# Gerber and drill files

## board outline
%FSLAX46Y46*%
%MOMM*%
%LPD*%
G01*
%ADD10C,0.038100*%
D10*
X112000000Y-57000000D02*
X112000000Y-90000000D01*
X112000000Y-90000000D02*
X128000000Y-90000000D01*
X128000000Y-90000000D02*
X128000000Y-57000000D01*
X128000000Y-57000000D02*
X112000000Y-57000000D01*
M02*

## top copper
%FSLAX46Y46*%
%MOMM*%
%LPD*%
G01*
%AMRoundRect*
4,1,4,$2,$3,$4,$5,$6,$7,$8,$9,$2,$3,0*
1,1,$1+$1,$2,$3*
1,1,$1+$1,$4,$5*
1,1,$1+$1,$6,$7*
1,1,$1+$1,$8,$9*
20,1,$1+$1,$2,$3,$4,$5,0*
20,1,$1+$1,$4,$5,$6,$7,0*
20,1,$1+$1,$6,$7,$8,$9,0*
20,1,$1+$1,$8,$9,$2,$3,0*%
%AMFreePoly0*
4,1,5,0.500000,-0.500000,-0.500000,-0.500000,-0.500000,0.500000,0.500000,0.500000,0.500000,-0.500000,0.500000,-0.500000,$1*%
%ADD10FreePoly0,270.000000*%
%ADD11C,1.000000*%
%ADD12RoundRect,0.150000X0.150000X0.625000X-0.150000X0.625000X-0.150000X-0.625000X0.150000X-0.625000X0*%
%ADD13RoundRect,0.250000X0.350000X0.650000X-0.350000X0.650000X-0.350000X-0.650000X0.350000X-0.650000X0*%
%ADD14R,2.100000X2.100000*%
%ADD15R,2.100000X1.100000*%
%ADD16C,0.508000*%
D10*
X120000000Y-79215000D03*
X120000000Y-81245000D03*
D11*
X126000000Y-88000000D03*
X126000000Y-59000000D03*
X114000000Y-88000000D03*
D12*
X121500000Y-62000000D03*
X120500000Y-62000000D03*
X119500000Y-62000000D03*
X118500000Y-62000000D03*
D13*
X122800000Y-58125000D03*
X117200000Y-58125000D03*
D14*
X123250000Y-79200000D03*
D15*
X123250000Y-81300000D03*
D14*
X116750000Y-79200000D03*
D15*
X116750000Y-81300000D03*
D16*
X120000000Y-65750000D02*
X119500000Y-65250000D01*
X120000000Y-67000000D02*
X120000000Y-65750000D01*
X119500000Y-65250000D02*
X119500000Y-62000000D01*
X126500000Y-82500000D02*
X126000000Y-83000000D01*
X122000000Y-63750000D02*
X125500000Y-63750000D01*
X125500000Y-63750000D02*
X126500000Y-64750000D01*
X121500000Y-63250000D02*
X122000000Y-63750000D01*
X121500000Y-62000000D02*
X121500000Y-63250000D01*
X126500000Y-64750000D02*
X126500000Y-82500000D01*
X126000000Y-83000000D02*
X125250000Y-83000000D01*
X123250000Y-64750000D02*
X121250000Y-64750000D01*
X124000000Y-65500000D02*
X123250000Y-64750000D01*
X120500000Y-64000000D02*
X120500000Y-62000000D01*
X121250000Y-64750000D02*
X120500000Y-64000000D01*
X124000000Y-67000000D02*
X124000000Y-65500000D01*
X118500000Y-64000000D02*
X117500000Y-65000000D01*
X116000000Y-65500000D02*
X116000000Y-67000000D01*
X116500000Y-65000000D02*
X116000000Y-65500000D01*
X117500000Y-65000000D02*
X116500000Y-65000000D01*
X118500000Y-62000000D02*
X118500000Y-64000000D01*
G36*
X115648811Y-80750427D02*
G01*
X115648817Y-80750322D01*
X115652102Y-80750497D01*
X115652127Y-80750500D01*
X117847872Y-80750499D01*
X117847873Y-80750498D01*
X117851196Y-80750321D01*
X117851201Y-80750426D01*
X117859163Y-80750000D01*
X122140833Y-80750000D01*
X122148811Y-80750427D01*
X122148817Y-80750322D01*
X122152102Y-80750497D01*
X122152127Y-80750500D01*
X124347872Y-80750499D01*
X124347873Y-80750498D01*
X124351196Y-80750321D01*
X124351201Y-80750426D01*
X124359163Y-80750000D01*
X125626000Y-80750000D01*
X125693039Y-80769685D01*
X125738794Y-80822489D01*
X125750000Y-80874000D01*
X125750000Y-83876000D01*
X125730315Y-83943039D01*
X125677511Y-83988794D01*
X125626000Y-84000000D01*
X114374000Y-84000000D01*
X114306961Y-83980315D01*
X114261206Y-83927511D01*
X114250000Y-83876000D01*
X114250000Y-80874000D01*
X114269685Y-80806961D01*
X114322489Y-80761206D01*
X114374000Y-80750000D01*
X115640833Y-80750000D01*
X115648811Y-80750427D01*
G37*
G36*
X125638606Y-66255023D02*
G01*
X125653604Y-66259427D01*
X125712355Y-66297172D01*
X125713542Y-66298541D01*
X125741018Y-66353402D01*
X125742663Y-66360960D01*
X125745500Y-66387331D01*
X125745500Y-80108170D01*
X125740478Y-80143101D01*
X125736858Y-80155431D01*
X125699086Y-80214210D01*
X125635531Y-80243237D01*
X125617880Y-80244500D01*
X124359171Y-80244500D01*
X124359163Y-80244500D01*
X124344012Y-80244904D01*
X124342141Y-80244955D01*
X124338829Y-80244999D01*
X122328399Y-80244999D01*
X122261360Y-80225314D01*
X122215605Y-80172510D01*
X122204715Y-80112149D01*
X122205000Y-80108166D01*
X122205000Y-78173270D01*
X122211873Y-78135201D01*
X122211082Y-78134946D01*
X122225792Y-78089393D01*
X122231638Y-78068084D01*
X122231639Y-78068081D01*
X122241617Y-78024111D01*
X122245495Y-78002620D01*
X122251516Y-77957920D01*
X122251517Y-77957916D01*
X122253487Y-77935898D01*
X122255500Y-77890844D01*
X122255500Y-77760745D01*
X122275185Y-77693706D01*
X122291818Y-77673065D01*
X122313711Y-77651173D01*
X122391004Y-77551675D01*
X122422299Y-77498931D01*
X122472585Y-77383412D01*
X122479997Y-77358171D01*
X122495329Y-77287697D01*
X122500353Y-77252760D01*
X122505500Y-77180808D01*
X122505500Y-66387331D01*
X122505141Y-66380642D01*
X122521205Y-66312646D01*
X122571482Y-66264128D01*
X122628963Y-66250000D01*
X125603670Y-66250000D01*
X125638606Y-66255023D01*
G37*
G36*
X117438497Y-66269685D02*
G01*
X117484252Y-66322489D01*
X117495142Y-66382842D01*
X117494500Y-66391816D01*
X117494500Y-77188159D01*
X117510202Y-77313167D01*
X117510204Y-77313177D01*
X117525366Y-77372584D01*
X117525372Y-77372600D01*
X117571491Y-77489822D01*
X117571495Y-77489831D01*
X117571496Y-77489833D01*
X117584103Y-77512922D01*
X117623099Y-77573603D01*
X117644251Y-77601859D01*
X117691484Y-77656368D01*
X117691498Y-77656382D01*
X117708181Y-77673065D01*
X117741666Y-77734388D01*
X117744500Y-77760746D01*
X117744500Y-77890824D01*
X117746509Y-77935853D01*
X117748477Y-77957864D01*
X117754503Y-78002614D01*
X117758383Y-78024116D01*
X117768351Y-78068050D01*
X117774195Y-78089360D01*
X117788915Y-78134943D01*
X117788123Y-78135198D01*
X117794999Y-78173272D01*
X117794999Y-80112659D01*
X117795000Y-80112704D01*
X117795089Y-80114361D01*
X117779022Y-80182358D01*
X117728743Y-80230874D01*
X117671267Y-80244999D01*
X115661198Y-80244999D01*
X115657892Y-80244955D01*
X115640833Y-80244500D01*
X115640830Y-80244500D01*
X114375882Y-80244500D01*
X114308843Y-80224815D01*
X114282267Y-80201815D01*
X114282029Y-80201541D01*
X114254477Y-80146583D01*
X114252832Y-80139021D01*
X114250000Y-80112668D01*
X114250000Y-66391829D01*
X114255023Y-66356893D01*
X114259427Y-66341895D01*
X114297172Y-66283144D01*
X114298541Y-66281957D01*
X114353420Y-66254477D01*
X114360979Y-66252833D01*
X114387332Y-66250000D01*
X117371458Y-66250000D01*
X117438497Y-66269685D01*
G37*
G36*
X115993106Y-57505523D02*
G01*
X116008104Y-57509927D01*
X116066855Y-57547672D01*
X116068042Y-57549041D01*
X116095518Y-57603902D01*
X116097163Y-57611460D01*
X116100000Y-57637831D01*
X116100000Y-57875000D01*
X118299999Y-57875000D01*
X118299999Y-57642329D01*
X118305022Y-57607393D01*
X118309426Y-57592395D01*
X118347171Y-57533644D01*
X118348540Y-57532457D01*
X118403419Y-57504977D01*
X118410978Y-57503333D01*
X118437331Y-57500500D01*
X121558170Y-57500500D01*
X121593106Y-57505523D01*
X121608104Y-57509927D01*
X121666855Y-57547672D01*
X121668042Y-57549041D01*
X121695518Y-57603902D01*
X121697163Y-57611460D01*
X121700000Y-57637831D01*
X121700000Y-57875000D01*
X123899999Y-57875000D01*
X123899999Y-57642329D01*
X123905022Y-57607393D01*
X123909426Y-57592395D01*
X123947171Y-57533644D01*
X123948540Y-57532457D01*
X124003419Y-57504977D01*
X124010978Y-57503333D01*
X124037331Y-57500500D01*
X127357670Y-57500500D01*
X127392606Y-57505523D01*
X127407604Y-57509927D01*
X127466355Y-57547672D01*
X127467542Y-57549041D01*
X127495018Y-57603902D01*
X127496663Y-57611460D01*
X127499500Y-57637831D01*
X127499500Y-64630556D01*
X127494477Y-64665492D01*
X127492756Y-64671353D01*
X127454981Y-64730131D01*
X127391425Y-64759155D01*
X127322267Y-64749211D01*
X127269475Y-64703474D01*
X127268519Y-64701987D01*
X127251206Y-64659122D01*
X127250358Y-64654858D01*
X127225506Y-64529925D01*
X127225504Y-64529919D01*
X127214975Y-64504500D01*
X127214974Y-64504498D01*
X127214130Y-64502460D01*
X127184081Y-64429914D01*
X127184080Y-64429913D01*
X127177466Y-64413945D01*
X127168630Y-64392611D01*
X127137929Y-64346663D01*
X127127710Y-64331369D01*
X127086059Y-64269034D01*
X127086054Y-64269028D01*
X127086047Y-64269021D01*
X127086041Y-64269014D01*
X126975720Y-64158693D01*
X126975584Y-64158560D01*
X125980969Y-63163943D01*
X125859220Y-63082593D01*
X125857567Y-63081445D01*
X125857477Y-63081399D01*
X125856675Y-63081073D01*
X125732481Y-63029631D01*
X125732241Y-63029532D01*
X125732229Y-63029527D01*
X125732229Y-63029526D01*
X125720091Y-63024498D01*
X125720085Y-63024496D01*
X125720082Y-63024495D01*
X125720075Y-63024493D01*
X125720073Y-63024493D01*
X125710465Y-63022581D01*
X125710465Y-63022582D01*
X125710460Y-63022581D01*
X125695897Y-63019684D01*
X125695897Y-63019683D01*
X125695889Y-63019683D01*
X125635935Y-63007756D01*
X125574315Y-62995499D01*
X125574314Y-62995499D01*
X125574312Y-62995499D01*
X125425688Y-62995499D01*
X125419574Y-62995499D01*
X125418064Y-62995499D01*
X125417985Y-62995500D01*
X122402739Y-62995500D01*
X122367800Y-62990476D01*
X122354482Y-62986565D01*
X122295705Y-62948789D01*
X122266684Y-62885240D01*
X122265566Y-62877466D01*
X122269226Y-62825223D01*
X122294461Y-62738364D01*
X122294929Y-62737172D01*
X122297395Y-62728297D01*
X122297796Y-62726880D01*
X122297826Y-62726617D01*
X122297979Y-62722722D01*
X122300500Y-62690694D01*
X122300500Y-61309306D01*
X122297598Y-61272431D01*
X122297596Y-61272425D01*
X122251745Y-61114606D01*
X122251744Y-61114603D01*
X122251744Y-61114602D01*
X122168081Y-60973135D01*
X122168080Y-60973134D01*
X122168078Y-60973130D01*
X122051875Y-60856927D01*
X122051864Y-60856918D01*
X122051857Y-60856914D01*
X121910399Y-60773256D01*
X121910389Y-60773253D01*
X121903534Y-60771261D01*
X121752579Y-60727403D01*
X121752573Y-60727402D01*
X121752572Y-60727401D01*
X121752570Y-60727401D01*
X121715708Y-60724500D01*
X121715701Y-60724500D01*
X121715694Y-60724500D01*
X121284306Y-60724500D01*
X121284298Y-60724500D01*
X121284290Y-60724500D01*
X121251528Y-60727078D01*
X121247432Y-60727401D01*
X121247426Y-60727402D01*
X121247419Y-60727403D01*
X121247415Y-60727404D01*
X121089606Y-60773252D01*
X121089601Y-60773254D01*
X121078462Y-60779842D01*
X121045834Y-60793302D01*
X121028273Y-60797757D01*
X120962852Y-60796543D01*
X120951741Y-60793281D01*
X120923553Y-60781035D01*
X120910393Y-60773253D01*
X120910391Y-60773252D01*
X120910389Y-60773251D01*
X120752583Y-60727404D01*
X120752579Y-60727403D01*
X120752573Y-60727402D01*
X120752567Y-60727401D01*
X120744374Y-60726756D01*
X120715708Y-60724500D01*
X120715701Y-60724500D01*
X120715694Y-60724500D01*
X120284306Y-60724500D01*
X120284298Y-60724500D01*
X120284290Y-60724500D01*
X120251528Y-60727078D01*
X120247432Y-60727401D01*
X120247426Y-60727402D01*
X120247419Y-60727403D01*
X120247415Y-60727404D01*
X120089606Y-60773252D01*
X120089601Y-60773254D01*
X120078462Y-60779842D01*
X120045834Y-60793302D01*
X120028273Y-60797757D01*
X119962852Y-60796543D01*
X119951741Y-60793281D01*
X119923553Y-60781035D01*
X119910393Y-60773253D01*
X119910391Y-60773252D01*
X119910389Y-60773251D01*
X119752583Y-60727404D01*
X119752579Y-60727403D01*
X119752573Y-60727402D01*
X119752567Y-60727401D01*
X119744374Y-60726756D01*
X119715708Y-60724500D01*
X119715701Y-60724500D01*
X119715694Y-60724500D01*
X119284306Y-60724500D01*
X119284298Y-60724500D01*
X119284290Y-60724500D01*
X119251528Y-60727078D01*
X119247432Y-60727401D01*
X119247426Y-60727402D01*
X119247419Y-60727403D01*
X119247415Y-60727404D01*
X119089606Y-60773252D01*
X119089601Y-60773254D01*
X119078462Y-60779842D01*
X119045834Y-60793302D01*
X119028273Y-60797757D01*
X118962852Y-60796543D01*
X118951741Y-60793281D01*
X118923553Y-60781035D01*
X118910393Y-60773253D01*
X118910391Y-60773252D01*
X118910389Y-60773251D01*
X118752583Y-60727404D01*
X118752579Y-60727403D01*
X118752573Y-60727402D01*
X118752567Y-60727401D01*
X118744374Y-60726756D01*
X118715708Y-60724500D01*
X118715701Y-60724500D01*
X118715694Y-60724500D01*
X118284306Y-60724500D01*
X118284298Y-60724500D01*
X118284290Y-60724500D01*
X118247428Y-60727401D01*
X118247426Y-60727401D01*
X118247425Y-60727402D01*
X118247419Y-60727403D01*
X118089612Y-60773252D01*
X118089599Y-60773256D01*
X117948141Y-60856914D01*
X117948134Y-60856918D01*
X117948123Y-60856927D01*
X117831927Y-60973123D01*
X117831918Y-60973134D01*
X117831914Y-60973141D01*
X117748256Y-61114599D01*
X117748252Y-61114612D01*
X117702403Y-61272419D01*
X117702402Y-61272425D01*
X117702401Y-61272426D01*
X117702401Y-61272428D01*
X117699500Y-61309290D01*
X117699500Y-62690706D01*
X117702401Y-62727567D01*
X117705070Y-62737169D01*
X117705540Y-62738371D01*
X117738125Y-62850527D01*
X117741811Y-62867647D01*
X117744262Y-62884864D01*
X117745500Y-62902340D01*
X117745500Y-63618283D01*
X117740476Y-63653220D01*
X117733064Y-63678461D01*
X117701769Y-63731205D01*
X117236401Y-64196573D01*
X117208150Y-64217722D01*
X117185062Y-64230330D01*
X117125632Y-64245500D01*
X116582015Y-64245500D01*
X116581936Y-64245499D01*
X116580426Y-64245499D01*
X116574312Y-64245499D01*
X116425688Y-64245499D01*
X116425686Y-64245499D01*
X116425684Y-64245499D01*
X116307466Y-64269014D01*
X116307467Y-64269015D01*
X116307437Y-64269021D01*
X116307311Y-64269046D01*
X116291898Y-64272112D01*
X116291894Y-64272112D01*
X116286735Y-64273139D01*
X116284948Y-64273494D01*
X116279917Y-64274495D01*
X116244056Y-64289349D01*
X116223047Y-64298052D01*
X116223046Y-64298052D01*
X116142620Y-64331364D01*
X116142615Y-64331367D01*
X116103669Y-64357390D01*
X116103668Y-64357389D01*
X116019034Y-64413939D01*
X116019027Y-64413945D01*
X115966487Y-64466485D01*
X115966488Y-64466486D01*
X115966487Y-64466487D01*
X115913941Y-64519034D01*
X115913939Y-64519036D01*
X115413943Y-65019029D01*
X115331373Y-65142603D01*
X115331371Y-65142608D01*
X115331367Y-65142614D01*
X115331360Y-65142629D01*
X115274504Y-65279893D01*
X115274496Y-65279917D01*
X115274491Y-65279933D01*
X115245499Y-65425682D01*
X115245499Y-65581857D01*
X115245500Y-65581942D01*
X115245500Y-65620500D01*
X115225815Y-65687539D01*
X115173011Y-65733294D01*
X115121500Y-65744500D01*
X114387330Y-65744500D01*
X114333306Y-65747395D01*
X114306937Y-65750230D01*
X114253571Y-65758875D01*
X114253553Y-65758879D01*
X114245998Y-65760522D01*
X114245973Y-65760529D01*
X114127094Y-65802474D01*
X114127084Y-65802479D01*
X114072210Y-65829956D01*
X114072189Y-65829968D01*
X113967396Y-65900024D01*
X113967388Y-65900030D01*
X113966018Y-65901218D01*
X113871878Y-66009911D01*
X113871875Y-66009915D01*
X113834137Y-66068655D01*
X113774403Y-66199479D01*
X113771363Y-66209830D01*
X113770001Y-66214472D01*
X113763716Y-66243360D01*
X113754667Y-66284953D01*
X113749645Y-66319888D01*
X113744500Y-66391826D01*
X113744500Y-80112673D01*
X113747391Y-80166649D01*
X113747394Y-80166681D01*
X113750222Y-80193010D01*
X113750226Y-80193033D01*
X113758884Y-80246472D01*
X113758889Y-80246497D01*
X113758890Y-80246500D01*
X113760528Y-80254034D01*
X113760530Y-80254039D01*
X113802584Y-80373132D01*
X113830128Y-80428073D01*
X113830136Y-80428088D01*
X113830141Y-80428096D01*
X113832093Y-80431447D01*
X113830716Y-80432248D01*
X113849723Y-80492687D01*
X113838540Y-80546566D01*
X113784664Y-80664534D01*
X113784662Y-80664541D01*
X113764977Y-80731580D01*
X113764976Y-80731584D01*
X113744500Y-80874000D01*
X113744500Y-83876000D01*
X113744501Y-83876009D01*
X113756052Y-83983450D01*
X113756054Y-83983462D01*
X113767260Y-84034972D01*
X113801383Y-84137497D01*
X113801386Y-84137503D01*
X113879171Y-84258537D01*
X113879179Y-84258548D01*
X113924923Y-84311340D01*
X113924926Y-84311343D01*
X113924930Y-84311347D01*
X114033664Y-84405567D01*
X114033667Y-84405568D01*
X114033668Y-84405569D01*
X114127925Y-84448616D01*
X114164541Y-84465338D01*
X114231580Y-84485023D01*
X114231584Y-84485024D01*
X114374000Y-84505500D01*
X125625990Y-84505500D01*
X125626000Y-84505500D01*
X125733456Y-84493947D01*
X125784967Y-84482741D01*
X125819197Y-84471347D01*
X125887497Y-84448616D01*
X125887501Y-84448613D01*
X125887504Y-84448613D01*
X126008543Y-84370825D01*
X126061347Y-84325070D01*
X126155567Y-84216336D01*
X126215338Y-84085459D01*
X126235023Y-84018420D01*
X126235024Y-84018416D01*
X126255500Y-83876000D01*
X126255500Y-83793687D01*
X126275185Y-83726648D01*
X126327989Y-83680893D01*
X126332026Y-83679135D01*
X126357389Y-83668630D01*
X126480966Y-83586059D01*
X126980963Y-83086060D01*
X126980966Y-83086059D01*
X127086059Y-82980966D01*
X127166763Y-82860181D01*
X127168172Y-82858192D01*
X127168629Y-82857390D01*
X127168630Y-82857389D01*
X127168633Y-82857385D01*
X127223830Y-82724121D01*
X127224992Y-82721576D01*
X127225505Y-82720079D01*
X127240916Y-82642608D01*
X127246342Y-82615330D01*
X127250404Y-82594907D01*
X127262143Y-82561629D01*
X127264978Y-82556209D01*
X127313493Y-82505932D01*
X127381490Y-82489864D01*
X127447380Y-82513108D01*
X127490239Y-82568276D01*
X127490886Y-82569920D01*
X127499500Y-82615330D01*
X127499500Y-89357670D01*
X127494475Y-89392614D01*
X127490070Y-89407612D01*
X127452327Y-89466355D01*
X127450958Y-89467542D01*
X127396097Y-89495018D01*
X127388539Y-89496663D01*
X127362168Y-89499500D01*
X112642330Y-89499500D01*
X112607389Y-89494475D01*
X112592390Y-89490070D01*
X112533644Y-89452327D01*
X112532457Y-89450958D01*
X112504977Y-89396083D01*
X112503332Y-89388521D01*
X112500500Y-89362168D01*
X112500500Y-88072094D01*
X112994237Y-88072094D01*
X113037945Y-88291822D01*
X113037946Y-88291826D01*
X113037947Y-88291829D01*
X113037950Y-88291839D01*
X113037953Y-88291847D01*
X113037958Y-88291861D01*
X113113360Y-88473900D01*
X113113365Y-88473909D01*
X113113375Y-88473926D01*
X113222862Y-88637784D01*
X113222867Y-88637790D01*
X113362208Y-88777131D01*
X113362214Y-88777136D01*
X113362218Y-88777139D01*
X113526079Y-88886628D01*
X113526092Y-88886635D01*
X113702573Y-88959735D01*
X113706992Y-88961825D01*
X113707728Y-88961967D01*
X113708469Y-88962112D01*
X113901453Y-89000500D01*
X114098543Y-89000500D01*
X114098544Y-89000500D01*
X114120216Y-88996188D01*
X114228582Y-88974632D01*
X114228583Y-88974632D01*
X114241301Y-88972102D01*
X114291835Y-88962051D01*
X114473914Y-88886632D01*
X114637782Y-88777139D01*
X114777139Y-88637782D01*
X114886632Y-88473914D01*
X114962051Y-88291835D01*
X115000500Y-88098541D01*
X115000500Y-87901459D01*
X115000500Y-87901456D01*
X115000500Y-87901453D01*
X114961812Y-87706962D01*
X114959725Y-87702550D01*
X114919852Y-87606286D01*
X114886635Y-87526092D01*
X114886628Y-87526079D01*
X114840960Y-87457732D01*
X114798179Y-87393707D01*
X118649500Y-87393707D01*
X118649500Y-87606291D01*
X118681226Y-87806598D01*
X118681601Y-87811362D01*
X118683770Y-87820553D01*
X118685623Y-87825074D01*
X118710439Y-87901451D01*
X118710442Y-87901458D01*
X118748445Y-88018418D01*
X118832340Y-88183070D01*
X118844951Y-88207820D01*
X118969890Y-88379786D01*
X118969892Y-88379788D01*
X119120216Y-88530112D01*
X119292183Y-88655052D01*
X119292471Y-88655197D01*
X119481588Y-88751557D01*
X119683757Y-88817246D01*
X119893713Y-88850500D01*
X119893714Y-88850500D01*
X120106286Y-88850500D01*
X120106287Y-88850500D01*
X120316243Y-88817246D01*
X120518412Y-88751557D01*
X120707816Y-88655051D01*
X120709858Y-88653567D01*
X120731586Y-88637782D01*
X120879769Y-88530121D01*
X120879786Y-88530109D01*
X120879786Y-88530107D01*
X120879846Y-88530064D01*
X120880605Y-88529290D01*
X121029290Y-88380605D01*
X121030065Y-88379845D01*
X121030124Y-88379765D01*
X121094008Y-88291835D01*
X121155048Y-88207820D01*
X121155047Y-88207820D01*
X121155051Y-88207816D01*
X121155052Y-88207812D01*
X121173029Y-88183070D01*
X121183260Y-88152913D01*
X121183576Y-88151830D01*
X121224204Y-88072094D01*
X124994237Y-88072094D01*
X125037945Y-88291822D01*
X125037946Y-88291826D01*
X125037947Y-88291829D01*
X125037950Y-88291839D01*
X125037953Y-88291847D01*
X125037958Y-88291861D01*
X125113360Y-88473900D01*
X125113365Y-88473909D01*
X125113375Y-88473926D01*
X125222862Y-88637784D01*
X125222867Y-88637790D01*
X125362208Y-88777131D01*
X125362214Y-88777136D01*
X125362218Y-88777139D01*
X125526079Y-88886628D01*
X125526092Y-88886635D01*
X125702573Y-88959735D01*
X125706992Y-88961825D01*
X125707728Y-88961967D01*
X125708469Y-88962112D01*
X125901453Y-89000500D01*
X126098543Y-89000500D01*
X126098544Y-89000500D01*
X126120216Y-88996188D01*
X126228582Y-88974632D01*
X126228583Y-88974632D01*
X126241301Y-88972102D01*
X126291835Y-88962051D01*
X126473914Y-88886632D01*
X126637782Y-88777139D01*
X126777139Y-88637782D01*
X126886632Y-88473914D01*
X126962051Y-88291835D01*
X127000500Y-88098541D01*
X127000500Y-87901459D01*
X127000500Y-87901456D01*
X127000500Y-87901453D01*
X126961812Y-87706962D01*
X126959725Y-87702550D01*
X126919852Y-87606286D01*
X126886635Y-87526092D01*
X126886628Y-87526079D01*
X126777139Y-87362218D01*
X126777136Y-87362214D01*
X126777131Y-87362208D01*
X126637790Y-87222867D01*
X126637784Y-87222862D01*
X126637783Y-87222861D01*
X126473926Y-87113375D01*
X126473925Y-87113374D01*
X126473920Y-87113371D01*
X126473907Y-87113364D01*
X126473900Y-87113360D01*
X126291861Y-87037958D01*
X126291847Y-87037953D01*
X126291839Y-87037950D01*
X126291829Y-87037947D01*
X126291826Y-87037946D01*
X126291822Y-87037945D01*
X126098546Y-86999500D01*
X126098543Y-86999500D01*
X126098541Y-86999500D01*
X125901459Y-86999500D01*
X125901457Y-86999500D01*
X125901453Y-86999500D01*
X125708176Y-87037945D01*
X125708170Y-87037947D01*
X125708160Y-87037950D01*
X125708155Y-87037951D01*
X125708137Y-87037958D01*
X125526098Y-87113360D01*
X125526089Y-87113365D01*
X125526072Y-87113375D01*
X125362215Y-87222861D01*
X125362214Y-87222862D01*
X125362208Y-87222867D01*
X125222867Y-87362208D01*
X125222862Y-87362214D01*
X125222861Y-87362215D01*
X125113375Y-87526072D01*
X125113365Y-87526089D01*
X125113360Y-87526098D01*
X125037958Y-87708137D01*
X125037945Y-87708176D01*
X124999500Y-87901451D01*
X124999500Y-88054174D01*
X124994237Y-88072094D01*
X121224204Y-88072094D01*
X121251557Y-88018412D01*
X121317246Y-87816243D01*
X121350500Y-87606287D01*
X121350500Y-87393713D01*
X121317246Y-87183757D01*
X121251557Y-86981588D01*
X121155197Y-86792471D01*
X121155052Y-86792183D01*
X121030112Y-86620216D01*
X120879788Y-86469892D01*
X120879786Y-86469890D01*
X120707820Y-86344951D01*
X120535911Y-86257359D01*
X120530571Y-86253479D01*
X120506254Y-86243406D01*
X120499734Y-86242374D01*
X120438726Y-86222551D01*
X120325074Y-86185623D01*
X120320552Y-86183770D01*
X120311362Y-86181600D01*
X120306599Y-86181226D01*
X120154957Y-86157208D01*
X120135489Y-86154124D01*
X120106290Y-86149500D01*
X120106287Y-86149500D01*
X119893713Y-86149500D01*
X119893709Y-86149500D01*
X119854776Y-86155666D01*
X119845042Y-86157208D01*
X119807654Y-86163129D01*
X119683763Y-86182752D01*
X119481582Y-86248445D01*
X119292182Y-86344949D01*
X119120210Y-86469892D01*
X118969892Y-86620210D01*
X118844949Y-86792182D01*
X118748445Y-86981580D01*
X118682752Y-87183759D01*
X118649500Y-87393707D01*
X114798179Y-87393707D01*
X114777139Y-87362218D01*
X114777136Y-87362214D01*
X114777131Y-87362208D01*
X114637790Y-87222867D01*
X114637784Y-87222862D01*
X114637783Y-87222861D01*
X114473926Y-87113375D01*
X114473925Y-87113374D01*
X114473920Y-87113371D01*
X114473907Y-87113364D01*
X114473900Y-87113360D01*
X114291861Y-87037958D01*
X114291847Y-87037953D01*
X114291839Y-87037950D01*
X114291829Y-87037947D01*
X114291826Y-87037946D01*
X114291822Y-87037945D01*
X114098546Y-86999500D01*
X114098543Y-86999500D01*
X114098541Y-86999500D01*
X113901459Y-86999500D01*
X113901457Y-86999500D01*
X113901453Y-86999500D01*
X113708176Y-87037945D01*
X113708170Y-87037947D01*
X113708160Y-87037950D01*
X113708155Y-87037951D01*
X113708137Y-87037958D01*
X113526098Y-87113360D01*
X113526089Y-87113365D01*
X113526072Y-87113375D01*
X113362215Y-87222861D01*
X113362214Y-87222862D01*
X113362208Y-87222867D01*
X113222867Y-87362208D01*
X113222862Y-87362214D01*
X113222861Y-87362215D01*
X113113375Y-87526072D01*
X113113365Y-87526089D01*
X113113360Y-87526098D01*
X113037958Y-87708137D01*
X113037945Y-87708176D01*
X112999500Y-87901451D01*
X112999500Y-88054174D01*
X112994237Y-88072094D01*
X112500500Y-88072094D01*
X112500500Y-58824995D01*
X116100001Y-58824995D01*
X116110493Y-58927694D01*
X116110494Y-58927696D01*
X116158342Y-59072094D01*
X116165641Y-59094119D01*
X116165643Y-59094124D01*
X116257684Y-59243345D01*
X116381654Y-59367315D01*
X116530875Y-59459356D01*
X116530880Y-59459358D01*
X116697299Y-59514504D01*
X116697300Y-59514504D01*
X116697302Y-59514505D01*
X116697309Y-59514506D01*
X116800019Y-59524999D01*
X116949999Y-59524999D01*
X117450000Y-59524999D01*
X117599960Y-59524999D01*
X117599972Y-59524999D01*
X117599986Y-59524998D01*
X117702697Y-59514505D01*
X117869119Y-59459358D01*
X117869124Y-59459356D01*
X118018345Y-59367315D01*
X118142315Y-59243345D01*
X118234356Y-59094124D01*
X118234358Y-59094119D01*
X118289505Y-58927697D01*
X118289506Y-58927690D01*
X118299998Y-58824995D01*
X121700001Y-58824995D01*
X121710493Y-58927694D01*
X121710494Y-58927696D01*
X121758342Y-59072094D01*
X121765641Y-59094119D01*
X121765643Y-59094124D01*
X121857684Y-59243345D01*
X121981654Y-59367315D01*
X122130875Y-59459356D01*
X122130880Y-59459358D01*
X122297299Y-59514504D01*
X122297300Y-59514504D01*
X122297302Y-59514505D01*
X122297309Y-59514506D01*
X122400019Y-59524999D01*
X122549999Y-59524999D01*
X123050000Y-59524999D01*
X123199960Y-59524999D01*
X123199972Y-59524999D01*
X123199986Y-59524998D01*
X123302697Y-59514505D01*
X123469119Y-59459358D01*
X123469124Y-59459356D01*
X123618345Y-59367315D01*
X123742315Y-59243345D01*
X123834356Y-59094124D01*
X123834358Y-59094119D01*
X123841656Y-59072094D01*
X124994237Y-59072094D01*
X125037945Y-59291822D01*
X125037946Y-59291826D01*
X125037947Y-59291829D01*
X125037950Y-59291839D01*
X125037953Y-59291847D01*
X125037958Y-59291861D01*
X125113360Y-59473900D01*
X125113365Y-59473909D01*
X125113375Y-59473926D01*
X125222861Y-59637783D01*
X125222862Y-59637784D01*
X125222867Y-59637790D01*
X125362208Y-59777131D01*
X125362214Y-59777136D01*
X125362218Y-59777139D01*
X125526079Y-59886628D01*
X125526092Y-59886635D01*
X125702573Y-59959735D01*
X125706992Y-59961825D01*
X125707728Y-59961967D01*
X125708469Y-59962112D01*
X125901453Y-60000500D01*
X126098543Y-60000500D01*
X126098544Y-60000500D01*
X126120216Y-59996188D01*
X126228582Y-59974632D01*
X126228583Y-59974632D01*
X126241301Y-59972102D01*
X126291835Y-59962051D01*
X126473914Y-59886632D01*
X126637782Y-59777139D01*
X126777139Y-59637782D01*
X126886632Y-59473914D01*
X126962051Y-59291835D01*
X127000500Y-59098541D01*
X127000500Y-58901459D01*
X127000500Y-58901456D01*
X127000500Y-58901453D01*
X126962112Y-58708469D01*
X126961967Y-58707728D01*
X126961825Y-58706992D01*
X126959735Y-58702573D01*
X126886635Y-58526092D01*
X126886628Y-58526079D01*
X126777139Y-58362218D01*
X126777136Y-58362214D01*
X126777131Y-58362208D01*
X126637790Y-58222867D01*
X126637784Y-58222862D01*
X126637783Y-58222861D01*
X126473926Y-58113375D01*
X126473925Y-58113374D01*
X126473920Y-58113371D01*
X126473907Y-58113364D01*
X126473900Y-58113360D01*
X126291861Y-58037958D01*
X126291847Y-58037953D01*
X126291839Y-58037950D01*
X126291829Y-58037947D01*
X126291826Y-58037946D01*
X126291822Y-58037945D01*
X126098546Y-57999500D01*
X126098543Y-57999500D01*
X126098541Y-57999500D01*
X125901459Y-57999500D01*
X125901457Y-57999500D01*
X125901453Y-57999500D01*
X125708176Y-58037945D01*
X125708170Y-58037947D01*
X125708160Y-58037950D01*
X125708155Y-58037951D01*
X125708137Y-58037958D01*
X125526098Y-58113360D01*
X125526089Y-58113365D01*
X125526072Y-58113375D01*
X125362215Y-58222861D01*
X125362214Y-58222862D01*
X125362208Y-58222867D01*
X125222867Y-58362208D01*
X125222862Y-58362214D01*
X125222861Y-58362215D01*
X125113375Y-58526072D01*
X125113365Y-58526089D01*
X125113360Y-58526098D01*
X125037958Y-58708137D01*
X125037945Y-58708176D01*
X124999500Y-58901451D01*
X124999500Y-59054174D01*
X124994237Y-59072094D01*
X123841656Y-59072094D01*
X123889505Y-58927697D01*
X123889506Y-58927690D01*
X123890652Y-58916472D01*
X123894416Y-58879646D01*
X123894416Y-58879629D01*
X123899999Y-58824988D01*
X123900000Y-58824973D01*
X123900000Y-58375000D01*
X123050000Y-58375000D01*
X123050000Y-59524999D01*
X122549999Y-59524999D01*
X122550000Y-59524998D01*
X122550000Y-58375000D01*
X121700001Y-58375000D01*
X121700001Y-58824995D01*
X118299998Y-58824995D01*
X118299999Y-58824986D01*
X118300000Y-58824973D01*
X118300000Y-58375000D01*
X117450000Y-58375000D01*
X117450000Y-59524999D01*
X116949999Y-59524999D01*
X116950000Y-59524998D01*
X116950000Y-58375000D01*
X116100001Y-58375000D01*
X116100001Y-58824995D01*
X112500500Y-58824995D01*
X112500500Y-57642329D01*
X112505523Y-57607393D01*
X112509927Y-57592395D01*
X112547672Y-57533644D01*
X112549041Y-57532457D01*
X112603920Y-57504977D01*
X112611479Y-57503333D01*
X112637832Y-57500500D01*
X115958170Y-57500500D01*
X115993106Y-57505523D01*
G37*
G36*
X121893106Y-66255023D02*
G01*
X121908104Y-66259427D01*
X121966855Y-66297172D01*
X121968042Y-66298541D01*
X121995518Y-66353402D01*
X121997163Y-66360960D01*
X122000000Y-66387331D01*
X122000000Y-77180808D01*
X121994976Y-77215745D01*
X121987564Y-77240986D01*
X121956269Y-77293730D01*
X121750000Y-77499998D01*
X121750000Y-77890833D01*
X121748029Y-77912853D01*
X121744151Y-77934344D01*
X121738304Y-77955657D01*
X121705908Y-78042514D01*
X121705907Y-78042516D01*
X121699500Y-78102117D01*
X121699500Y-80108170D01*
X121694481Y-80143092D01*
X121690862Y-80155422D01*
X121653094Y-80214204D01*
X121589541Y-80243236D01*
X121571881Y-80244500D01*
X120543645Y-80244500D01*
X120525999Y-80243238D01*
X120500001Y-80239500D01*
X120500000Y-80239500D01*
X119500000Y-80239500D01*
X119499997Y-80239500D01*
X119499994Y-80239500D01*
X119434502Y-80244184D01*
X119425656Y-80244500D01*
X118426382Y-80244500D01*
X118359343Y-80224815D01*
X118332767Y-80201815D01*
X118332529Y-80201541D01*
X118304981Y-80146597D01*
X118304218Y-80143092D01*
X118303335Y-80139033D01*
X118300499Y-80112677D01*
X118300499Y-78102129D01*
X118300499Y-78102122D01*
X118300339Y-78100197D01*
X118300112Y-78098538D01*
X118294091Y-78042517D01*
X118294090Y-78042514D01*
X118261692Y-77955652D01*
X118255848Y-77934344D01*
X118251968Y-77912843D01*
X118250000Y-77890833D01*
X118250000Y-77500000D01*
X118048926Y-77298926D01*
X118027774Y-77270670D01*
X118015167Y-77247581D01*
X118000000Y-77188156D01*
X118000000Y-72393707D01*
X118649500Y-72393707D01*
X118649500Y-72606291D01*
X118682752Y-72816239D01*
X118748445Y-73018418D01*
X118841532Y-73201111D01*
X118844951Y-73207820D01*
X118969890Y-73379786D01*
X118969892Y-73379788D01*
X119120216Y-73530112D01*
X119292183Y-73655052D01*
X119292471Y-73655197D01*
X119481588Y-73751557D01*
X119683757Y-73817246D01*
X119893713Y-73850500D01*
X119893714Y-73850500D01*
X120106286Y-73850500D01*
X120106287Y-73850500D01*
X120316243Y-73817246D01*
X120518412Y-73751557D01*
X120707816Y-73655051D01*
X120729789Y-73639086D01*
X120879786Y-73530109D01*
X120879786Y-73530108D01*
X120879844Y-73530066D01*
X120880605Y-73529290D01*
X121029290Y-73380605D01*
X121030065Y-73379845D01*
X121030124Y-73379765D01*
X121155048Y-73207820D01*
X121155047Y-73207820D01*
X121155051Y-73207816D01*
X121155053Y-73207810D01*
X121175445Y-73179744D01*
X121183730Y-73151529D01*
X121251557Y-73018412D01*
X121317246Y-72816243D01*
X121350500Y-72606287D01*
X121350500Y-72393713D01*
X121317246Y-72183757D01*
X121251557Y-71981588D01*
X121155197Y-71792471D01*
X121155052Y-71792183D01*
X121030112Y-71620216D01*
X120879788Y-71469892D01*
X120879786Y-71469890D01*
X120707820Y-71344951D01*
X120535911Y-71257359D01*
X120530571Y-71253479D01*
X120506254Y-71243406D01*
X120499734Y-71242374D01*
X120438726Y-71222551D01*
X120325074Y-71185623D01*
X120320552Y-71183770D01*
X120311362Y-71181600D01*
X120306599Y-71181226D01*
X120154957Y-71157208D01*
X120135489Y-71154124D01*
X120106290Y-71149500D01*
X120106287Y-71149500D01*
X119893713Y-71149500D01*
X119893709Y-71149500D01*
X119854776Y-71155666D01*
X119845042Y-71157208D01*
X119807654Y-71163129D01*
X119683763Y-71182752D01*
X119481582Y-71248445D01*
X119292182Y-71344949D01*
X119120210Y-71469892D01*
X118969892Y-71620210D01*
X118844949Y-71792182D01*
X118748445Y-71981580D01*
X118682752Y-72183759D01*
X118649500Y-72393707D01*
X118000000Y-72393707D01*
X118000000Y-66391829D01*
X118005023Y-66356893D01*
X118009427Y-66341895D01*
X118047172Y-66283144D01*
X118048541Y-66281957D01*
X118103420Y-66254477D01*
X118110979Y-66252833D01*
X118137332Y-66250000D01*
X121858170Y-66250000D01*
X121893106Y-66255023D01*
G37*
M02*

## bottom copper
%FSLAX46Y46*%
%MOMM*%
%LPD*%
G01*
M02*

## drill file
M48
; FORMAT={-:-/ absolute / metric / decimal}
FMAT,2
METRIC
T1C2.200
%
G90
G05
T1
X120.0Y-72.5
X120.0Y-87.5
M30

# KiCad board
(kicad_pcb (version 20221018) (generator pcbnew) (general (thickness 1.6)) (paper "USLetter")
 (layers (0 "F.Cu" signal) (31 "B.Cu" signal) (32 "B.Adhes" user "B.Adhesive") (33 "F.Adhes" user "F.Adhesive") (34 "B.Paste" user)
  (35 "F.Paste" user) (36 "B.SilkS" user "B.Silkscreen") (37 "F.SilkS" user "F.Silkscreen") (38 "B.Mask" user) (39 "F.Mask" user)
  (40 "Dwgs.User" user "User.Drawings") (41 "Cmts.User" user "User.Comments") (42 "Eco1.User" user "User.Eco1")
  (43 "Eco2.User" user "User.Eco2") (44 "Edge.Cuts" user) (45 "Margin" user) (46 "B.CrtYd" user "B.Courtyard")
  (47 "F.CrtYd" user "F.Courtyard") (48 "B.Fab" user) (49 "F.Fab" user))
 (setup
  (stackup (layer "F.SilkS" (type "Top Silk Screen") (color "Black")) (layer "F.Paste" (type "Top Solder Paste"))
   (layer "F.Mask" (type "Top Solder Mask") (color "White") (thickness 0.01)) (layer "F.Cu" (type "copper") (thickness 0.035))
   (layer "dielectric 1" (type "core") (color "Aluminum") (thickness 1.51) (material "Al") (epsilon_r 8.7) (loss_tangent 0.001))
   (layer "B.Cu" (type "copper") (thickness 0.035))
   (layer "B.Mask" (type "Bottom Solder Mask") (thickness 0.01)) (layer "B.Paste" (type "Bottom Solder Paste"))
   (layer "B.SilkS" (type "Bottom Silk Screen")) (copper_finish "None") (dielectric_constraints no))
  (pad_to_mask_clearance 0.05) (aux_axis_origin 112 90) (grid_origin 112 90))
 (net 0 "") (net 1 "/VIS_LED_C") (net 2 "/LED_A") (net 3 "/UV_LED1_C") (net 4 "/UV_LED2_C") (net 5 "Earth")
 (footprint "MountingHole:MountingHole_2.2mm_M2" (layer "F.Cu") (at 120 87.5)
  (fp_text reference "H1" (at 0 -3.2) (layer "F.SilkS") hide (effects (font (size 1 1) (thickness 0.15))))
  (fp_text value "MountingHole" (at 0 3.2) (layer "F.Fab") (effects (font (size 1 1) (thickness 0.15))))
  (pad "" np_thru_hole circle (at 0 0) (size 2.2 2.2) (drill 2.2) (layers "*.Cu" "*.Mask")))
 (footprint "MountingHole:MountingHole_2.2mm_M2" (layer "F.Cu") (at 120 72.5)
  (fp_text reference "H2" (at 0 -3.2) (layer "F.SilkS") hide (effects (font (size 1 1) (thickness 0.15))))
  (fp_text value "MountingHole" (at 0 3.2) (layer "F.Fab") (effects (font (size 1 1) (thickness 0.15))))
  (pad "" np_thru_hole circle (at 0 0) (size 2.2 2.2) (drill 2.2) (layers "*.Cu" "*.Mask")))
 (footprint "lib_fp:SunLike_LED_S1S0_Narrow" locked (layer "F.Cu") (at 120 80 -90) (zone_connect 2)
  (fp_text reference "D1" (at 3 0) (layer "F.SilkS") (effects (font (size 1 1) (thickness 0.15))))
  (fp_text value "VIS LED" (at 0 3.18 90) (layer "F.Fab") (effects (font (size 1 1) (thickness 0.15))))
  (pad "1" smd custom locked (at -0.785 0 270) (size 1 1) (layers "F.Cu" "F.Paste" "F.Mask") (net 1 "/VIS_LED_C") (zone_connect 2)
   (thermal_bridge_angle 45) (options (clearance outline) (anchor rect)) (primitives))
  (pad "2" smd custom locked (at 1.245 0 270) (size 1 1) (layers "F.Cu" "F.Paste" "F.Mask") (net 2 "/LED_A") (zone_connect 2)
   (thermal_bridge_angle 45) (options (clearance outline) (anchor rect)) (primitives)))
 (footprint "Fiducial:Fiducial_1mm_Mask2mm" (layer "F.Cu") (at 126 88 90)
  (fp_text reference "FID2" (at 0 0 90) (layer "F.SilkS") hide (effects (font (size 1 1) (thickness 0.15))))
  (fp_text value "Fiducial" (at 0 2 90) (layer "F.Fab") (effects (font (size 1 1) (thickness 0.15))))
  (pad "" smd circle (at 0 0 90) (size 1 1) (layers "F.Cu" "F.Mask") (solder_mask_margin 0.5) (clearance 0.5)))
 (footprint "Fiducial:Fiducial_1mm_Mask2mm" (layer "F.Cu") (at 126 59 90)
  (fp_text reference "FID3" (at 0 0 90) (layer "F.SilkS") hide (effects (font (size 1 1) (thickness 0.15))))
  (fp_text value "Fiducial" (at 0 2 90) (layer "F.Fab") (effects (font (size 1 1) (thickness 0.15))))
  (pad "" smd circle (at 0 0 90) (size 1 1) (layers "F.Cu" "F.Mask") (solder_mask_margin 0.5) (clearance 0.5)))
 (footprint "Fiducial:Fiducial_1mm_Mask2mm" (layer "F.Cu") (at 114 88 90)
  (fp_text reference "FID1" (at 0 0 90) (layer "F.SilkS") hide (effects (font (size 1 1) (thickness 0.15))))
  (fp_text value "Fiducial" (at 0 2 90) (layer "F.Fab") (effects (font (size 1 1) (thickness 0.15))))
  (pad "" smd circle (at 0 0 90) (size 1 1) (layers "F.Cu" "F.Mask") (solder_mask_margin 0.5) (clearance 0.5)))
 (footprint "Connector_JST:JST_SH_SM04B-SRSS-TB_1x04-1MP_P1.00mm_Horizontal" (layer "F.Cu") (at 120 60 180)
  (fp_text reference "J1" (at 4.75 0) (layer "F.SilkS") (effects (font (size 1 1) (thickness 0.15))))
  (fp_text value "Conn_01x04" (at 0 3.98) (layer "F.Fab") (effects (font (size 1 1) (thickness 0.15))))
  (pad "1" smd roundrect (at -1.5 -2 180) (size 0.6 1.55) (layers "F.Cu" "F.Paste" "F.Mask") (roundrect_rratio 0.25) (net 2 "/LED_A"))
  (pad "2" smd roundrect (at -0.5 -2 180) (size 0.6 1.55) (layers "F.Cu" "F.Paste" "F.Mask") (roundrect_rratio 0.25) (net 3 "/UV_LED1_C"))
  (pad "3" smd roundrect (at 0.5 -2 180) (size 0.6 1.55) (layers "F.Cu" "F.Paste" "F.Mask") (roundrect_rratio 0.25) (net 1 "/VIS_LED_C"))
  (pad "4" smd roundrect (at 1.5 -2 180) (size 0.6 1.55) (layers "F.Cu" "F.Paste" "F.Mask") (roundrect_rratio 0.25) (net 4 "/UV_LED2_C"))
  (pad "MP" smd roundrect (at -2.8 1.875 180) (size 1.2 1.8) (layers "F.Cu" "F.Paste" "F.Mask") (roundrect_rratio 0.2083333333)
   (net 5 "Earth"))
  (pad "MP" smd roundrect (at 2.8 1.875 180) (size 1.2 1.8) (layers "F.Cu" "F.Paste" "F.Mask") (roundrect_rratio 0.2083333333)
   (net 5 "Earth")))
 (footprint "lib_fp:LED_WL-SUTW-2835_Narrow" (layer "F.Cu") (at 123.25 80 -90) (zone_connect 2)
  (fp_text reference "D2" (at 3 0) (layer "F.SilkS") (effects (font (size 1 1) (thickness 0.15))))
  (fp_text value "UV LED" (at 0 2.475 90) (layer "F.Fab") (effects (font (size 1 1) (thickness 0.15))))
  (pad "1" smd rect (at -0.8 0 270) (size 2.1 2.1) (layers "F.Cu" "F.Paste" "F.Mask") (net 3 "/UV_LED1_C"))
  (pad "2" smd rect (at 1.3 0 270) (size 1.1 2.1) (layers "F.Cu" "F.Paste" "F.Mask") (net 2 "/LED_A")))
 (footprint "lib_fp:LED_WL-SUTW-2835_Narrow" (layer "F.Cu") (at 116.75 80 -90) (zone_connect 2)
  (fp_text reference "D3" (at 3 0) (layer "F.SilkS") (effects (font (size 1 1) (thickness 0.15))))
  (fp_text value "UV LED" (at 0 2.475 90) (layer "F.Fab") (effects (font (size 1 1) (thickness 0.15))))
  (pad "1" smd rect (at -0.8 0 270) (size 2.1 2.1) (layers "F.Cu" "F.Paste" "F.Mask") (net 4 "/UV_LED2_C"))
  (pad "2" smd rect (at 1.3 0 270) (size 1.1 2.1) (layers "F.Cu" "F.Paste" "F.Mask") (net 2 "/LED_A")))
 (gr_line (start 112 57) (end 112 90) (stroke (width 0.0381) (type solid)) (layer "Edge.Cuts"))
 (gr_line (start 112 90) (end 128 90) (stroke (width 0.0381) (type solid)) (layer "Edge.Cuts"))
 (gr_line (start 128 90) (end 128 57) (stroke (width 0.0381) (type solid)) (layer "Edge.Cuts"))
 (gr_line (start 128 57) (end 112 57) (stroke (width 0.0381) (type solid)) (layer "Edge.Cuts"))
 (segment (start 120 65.75) (end 119.5 65.25) (width 0.508) (layer "F.Cu") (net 1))
 (segment (start 120 67) (end 120 65.75) (width 0.508) (layer "F.Cu") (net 1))
 (segment (start 119.5 65.25) (end 119.5 62) (width 0.508) (layer "F.Cu") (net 1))
 (segment (start 126.5 82.5) (end 126 83) (width 0.508) (layer "F.Cu") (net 2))
 (segment (start 122 63.75) (end 125.5 63.75) (width 0.508) (layer "F.Cu") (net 2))
 (segment (start 125.5 63.75) (end 126.5 64.75) (width 0.508) (layer "F.Cu") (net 2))
 (segment (start 121.5 63.25) (end 122 63.75) (width 0.508) (layer "F.Cu") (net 2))
 (segment (start 121.5 62) (end 121.5 63.25) (width 0.508) (layer "F.Cu") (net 2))
 (segment (start 126.5 64.75) (end 126.5 82.5) (width 0.508) (layer "F.Cu") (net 2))
 (segment (start 126 83) (end 125.25 83) (width 0.508) (layer "F.Cu") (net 2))
 (segment (start 123.25 64.75) (end 121.25 64.75) (width 0.508) (layer "F.Cu") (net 3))
 (segment (start 124 65.5) (end 123.25 64.75) (width 0.508) (layer "F.Cu") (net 3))
 (segment (start 120.5 64) (end 120.5 62) (width 0.508) (layer "F.Cu") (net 3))
 (segment (start 121.25 64.75) (end 120.5 64) (width 0.508) (layer "F.Cu") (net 3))
 (segment (start 124 67) (end 124 65.5) (width 0.508) (layer "F.Cu") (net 3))
 (segment (start 118.5 64) (end 117.5 65) (width 0.508) (layer "F.Cu") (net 4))
 (segment (start 116 65.5) (end 116 67) (width 0.508) (layer "F.Cu") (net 4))
 (segment (start 116.5 65) (end 116 65.5) (width 0.508) (layer "F.Cu") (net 4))
 (segment (start 117.5 65) (end 116.5 65) (width 0.508) (layer "F.Cu") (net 4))
 (segment (start 118.5 62) (end 118.5 64) (width 0.508) (layer "F.Cu") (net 4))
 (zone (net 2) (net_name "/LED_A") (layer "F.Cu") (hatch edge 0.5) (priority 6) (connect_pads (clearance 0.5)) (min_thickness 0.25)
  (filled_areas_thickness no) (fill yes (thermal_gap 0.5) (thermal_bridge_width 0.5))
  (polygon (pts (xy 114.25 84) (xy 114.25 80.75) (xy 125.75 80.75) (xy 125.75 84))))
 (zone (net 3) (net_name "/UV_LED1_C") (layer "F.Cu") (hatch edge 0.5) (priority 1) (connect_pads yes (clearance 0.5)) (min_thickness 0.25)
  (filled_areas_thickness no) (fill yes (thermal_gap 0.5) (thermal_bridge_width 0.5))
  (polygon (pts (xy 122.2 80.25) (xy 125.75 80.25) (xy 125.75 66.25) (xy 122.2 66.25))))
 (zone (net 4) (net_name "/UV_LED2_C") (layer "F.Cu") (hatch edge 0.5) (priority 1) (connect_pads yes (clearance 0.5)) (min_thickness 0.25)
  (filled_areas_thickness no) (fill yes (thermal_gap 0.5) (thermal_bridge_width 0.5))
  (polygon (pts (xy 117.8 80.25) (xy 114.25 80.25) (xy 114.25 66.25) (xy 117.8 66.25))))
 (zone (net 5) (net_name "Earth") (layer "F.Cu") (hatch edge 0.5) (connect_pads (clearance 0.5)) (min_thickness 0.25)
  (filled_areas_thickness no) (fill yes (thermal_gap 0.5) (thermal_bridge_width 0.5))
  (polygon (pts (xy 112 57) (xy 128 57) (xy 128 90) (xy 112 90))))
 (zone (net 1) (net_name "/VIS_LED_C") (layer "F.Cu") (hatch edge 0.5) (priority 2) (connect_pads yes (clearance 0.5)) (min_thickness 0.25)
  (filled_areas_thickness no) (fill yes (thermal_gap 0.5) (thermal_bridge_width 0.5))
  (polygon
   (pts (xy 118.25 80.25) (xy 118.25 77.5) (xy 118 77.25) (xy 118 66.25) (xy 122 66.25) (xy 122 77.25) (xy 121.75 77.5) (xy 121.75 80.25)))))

